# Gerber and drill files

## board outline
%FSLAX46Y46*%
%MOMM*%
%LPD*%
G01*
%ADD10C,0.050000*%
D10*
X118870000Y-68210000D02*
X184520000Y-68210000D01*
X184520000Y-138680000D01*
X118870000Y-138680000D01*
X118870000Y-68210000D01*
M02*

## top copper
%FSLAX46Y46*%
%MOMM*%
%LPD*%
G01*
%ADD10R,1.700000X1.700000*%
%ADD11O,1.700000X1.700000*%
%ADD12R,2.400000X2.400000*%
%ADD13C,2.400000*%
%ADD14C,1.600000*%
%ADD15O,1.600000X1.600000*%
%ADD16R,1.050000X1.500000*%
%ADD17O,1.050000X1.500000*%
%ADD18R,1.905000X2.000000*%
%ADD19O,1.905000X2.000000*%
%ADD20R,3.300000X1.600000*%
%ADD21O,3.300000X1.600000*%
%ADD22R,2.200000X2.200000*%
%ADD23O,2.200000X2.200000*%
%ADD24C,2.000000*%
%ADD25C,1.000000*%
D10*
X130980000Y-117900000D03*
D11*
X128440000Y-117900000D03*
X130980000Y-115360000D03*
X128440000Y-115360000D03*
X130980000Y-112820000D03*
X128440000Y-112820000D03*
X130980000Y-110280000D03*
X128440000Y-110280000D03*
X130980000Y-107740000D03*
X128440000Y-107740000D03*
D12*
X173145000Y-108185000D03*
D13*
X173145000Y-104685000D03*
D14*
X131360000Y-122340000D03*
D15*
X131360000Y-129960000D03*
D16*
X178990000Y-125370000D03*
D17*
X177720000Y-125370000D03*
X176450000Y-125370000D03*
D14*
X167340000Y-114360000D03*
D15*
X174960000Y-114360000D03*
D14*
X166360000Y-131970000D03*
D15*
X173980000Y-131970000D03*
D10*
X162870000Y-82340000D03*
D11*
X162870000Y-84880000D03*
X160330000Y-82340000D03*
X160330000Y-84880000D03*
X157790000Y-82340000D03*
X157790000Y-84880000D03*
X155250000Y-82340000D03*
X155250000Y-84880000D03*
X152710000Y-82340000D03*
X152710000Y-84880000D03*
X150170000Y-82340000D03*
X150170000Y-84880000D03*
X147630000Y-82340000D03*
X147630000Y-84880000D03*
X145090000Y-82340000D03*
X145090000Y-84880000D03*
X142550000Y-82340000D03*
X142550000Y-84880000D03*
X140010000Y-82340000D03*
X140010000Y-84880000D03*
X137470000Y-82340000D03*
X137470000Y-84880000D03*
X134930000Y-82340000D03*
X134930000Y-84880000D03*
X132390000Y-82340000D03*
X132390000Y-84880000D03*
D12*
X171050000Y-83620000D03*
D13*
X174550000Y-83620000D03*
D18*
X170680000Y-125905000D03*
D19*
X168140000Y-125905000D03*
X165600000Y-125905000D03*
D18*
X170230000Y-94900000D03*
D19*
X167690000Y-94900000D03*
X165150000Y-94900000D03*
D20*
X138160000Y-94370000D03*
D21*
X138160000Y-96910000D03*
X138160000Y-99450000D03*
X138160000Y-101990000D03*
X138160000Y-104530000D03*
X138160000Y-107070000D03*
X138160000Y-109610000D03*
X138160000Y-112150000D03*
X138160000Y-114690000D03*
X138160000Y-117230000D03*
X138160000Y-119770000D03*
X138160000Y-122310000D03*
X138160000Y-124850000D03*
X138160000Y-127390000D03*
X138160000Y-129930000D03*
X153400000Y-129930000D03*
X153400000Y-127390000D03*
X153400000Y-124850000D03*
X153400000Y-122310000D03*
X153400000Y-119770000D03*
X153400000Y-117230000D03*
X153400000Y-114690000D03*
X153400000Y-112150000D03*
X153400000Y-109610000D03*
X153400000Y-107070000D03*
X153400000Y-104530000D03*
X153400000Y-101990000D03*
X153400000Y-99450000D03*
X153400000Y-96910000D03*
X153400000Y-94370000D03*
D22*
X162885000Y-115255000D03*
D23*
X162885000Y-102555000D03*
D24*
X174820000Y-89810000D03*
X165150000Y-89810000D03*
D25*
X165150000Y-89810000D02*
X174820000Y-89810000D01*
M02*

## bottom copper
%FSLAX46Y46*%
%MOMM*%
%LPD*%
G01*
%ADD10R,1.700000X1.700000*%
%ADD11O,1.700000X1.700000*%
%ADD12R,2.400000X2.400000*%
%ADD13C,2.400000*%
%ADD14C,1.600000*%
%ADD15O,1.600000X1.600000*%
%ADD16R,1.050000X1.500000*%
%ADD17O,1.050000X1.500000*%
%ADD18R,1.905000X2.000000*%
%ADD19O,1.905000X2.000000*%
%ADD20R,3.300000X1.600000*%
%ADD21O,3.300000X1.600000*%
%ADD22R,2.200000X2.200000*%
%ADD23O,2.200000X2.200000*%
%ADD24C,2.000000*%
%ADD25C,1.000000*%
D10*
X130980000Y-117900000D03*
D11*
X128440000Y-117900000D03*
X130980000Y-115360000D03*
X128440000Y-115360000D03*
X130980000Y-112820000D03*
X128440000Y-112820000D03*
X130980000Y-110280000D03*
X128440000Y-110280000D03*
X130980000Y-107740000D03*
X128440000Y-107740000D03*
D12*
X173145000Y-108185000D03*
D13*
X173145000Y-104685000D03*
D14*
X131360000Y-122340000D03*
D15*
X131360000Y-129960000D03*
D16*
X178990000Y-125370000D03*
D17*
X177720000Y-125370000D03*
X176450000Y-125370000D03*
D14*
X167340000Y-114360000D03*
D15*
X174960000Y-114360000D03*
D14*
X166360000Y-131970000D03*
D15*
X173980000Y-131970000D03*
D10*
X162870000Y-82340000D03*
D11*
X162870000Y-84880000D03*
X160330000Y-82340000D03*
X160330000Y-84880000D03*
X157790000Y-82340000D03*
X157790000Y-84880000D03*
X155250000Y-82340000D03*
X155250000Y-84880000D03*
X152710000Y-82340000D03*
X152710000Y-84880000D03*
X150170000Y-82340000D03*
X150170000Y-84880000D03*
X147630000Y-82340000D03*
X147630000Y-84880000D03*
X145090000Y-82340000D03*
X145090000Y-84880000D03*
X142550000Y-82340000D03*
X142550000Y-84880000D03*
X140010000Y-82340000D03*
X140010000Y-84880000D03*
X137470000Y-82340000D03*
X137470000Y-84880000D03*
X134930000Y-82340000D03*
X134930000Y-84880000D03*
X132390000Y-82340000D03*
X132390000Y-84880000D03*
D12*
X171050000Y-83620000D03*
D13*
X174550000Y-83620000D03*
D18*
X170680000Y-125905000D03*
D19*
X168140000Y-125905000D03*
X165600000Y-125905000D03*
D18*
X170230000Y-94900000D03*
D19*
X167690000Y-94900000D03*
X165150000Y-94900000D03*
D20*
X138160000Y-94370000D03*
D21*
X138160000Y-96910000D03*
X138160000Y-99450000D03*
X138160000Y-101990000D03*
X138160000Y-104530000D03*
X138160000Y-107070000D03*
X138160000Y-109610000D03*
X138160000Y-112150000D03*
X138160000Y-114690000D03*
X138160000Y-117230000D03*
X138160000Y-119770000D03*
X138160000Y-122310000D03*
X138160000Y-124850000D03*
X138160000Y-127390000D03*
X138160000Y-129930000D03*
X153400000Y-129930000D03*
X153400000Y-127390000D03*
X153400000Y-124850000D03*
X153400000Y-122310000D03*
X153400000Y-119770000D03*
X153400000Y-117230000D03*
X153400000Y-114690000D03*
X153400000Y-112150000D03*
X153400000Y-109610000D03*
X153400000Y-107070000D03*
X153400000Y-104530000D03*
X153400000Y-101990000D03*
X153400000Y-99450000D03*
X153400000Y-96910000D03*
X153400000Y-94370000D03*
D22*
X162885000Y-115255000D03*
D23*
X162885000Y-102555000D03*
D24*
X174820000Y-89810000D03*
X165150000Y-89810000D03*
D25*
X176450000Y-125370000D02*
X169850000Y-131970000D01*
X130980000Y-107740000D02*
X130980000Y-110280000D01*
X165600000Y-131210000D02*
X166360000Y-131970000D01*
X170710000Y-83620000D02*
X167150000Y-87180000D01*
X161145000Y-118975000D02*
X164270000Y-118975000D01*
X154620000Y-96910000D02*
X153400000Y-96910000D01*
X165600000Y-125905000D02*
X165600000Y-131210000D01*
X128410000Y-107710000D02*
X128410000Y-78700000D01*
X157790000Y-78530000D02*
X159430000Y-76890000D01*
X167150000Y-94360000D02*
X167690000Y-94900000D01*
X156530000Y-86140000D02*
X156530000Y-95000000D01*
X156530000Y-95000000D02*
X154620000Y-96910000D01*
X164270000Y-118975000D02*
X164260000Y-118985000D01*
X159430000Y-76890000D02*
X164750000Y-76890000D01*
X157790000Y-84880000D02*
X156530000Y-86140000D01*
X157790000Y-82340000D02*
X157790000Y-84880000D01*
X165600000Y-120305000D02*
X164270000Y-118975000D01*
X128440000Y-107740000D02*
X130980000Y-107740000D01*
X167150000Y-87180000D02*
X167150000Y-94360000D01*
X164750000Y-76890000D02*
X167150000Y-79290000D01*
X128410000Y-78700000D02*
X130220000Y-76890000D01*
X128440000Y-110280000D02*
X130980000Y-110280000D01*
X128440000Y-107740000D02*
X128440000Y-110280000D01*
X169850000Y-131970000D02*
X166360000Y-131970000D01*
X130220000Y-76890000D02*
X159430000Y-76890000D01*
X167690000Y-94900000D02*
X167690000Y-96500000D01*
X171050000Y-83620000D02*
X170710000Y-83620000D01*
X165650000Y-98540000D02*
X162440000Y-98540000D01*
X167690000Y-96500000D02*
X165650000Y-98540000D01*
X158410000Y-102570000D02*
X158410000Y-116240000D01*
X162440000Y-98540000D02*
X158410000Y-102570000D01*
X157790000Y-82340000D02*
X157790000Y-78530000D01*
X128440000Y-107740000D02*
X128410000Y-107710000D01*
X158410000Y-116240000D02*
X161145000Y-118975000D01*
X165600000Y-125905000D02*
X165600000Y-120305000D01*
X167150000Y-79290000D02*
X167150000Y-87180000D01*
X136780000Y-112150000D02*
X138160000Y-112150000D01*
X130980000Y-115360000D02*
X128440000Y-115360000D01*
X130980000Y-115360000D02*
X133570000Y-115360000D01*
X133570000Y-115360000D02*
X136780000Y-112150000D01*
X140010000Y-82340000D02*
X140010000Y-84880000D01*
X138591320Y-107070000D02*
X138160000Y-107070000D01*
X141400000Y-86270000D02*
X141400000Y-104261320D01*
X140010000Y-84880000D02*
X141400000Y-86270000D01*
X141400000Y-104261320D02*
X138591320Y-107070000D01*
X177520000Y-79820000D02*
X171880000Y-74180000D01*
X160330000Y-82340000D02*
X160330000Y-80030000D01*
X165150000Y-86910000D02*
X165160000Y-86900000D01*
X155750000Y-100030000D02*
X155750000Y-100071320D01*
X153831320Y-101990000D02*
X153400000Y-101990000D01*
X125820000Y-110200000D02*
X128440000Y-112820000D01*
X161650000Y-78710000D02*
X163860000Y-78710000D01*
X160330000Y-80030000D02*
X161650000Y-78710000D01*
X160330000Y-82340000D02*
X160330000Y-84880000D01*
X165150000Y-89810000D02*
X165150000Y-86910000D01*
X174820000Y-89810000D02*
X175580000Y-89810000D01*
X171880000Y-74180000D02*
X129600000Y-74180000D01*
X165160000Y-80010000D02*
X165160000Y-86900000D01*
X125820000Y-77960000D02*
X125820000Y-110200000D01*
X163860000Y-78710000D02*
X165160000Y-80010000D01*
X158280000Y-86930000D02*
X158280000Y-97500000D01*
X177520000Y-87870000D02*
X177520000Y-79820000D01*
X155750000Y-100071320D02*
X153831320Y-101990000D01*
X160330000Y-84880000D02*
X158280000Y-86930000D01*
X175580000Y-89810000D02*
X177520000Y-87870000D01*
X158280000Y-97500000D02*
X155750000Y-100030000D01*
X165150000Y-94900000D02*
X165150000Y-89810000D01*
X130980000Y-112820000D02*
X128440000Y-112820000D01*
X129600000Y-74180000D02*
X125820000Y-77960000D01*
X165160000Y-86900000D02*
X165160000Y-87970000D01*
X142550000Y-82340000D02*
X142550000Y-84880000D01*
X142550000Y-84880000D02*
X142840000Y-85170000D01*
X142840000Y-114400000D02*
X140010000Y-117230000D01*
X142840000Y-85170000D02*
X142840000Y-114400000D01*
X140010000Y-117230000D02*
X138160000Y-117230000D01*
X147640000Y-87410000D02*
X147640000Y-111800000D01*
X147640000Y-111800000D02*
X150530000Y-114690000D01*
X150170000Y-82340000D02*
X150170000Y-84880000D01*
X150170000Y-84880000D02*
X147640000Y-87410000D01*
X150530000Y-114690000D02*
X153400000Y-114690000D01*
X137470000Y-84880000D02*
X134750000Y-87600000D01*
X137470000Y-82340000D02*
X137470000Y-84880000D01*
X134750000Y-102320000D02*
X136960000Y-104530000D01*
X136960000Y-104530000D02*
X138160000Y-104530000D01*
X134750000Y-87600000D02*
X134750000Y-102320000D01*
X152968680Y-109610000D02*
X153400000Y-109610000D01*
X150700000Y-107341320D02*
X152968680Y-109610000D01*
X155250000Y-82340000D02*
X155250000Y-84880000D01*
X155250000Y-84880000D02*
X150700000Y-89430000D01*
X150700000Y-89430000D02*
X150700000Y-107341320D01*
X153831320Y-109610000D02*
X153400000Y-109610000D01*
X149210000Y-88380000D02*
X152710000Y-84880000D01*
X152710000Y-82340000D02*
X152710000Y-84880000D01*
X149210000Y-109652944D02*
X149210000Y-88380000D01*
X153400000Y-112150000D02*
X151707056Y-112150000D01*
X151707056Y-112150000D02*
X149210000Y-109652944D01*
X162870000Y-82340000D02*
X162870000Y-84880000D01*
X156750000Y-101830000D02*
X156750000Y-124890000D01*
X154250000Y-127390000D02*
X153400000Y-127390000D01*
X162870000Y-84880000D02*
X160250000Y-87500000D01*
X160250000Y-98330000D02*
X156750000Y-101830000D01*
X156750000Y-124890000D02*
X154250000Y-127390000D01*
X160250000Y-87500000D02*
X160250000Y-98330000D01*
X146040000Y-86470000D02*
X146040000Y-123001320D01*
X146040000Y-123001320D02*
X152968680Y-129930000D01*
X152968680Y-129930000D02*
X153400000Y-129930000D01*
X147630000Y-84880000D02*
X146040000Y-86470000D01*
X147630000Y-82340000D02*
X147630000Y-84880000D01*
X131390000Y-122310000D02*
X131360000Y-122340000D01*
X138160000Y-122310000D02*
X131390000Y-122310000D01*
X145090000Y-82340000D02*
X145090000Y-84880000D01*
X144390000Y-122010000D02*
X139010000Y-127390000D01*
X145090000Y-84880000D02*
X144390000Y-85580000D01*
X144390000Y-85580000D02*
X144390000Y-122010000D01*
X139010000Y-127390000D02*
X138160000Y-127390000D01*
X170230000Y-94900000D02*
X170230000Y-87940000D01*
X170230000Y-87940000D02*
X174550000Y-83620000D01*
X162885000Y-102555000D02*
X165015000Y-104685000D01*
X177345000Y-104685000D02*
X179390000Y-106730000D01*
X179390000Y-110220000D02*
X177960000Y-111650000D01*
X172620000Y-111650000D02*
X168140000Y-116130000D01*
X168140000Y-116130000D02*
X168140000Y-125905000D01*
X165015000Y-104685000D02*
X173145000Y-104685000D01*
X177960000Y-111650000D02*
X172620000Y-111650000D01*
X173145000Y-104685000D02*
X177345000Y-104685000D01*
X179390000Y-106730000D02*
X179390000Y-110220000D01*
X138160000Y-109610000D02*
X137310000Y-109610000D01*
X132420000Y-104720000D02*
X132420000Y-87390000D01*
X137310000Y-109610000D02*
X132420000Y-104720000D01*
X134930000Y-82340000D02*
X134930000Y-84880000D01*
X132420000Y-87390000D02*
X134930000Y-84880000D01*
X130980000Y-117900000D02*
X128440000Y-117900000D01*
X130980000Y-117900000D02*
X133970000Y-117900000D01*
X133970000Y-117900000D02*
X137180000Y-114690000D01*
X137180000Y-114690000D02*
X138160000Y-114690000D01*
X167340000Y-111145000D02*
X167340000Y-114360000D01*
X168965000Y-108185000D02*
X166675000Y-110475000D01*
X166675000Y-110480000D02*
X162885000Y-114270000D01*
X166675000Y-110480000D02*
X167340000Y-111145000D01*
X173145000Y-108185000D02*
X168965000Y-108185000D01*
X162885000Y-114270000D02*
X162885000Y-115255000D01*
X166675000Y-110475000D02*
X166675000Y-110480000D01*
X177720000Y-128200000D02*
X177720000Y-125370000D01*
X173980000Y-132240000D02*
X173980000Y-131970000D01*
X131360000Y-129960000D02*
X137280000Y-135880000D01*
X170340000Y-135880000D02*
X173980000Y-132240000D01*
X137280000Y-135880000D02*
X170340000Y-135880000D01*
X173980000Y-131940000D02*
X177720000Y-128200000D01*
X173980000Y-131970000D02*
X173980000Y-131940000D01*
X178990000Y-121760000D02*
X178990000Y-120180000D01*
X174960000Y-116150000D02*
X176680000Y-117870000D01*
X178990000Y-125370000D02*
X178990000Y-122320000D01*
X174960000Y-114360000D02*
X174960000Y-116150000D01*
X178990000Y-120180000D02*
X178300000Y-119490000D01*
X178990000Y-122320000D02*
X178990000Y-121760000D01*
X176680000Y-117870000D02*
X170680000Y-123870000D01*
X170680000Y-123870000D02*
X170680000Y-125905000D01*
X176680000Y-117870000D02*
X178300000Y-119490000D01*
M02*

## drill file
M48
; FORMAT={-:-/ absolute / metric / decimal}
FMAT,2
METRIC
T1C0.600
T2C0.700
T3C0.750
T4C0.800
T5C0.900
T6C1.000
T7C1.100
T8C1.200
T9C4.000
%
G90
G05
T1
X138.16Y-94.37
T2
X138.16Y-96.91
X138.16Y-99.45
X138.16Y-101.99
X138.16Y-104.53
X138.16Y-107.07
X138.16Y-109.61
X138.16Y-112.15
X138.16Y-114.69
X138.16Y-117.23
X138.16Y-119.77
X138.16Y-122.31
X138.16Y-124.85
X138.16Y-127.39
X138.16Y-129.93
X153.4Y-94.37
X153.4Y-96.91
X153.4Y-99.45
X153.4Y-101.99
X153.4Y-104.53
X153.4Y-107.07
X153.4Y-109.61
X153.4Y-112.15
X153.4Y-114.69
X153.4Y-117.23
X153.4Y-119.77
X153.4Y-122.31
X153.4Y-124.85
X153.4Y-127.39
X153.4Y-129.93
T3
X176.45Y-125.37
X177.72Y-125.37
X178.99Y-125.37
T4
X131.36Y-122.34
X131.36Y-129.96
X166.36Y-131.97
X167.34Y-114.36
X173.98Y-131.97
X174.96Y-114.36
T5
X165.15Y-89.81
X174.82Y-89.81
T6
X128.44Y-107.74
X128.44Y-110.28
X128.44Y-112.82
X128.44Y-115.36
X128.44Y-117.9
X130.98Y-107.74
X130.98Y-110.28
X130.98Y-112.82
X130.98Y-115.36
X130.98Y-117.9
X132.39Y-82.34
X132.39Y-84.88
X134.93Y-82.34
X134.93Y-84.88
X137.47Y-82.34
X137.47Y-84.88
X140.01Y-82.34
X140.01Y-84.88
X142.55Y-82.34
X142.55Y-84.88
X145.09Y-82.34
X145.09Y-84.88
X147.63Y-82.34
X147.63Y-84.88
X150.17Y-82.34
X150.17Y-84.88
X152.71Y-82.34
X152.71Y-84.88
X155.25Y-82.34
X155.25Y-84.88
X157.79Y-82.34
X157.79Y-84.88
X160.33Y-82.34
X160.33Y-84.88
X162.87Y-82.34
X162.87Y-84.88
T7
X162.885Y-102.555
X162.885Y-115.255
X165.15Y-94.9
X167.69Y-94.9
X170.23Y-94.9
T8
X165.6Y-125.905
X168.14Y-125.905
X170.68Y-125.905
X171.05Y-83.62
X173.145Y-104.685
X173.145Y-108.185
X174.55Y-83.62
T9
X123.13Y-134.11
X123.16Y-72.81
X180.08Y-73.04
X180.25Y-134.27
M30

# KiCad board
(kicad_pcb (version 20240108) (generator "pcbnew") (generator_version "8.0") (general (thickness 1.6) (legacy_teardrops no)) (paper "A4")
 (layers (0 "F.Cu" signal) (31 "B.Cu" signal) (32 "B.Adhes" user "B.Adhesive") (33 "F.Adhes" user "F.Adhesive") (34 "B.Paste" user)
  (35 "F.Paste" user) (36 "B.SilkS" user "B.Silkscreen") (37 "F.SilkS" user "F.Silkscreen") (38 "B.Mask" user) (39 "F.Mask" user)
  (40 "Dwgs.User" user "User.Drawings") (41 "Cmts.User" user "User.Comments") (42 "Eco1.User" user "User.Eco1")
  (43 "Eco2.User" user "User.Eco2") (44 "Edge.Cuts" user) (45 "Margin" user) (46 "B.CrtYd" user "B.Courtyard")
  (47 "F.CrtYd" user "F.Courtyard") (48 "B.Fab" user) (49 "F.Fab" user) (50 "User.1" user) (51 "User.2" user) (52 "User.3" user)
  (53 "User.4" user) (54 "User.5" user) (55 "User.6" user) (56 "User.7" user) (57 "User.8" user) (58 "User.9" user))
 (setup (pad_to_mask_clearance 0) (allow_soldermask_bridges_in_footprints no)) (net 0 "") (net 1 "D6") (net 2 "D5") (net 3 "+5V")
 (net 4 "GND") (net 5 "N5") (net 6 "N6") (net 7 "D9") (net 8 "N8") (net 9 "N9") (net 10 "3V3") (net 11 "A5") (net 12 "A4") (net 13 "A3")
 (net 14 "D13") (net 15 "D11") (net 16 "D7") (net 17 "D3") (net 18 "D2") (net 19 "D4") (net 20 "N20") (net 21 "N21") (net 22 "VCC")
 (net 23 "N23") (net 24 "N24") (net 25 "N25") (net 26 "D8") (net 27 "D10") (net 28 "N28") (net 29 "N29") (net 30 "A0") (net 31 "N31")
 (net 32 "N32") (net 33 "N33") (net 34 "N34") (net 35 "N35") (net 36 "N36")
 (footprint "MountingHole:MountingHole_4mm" (layer "F.Cu") (at 180.25 134.27)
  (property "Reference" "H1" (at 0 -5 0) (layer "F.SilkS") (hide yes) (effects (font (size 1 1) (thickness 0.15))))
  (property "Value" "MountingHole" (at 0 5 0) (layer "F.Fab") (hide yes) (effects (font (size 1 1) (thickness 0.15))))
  (pad "" np_thru_hole circle (at 0 0) (size 4 4) (drill 4) (layers "*.Cu" "*.Mask")))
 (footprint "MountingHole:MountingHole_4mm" (layer "F.Cu") (at 123.16 72.81)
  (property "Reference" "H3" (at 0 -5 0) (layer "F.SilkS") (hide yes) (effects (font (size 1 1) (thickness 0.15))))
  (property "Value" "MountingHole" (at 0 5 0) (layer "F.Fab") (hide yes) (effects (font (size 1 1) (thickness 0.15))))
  (pad "" np_thru_hole circle (at 0 0) (size 4 4) (drill 4) (layers "*.Cu" "*.Mask")))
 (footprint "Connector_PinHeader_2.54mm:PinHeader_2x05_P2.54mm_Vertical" (layer "F.Cu") (at 130.98 117.9 180)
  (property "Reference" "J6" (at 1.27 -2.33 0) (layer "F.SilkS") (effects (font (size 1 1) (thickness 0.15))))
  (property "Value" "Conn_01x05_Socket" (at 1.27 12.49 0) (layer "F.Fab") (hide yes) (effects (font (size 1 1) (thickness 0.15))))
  (pad "1" thru_hole rect (at 0 0 180) (size 1.7 1.7) (drill 1) (layers "*.Cu" "*.Mask") (remove_unused_layers no) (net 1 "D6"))
  (pad "1" thru_hole oval (at 2.54 0 180) (size 1.7 1.7) (drill 1) (layers "*.Cu" "*.Mask") (remove_unused_layers no) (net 1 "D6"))
  (pad "2" thru_hole oval (at 0 2.54 180) (size 1.7 1.7) (drill 1) (layers "*.Cu" "*.Mask") (remove_unused_layers no) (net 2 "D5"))
  (pad "2" thru_hole oval (at 2.54 2.54 180) (size 1.7 1.7) (drill 1) (layers "*.Cu" "*.Mask") (remove_unused_layers no) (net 2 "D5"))
  (pad "3" thru_hole oval (at 0 5.08 180) (size 1.7 1.7) (drill 1) (layers "*.Cu" "*.Mask") (remove_unused_layers no) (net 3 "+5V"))
  (pad "3" thru_hole oval (at 2.54 5.08 180) (size 1.7 1.7) (drill 1) (layers "*.Cu" "*.Mask") (remove_unused_layers no) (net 3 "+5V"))
  (pad "4" thru_hole oval (at 0 7.62 180) (size 1.7 1.7) (drill 1) (layers "*.Cu" "*.Mask") (remove_unused_layers no) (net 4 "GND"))
  (pad "4" thru_hole oval (at 2.54 7.62 180) (size 1.7 1.7) (drill 1) (layers "*.Cu" "*.Mask") (remove_unused_layers no) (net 4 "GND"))
  (pad "5" thru_hole oval (at 0 10.16 180) (size 1.7 1.7) (drill 1) (layers "*.Cu" "*.Mask") (remove_unused_layers no) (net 4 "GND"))
  (pad "5" thru_hole oval (at 2.54 10.16 180) (size 1.7 1.7) (drill 1) (layers "*.Cu" "*.Mask") (remove_unused_layers no) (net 4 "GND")))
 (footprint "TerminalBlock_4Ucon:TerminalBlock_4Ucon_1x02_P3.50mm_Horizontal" (layer "F.Cu") (at 173.145 108.185 90)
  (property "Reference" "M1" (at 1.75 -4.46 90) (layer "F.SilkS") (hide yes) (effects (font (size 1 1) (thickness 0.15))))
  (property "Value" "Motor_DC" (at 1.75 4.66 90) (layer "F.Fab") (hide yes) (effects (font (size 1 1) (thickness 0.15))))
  (pad "1" thru_hole rect (at 0 0 90) (size 2.4 2.4) (drill 1.2) (layers "*.Cu" "*.Mask") (remove_unused_layers no) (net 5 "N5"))
  (pad "2" thru_hole circle (at 3.5 0 90) (size 2.4 2.4) (drill 1.2) (layers "*.Cu" "*.Mask") (remove_unused_layers no) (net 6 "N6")))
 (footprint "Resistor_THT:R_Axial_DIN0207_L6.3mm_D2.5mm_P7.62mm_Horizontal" (layer "F.Cu") (at 131.36 122.34 -90)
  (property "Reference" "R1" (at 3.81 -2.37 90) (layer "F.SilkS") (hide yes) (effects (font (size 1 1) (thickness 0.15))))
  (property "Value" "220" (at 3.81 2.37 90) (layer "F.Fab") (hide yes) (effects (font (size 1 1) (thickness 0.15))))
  (pad "1" thru_hole circle (at 0 0 270) (size 1.6 1.6) (drill 0.8) (layers "*.Cu" "*.Mask") (remove_unused_layers no) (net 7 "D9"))
  (pad "2" thru_hole oval (at 7.62 0 270) (size 1.6 1.6) (drill 0.8) (layers "*.Cu" "*.Mask") (remove_unused_layers no) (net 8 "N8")))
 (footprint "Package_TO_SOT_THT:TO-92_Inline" (layer "F.Cu") (at 178.99 125.37 180)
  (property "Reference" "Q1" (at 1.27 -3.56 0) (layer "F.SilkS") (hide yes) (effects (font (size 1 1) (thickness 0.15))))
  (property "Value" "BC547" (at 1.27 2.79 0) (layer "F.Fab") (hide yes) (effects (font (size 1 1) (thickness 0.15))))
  (pad "1" thru_hole rect (at 0 0 180) (size 1.05 1.5) (drill 0.75) (layers "*.Cu" "*.Mask") (remove_unused_layers no) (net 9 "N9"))
  (pad "2" thru_hole oval (at 1.27 0 180) (size 1.05 1.5) (drill 0.75) (layers "*.Cu" "*.Mask") (remove_unused_layers no) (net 8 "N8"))
  (pad "3" thru_hole oval (at 2.54 0 180) (size 1.05 1.5) (drill 0.75) (layers "*.Cu" "*.Mask") (remove_unused_layers no) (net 4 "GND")))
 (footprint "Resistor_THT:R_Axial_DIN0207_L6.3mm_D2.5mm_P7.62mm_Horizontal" (layer "F.Cu") (at 167.34 114.36)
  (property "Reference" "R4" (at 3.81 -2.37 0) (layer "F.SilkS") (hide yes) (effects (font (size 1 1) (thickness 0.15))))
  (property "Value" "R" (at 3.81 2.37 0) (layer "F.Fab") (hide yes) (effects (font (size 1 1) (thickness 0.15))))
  (pad "1" thru_hole circle (at 0 0) (size 1.6 1.6) (drill 0.8) (layers "*.Cu" "*.Mask") (remove_unused_layers no) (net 5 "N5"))
  (pad "2" thru_hole oval (at 7.62 0) (size 1.6 1.6) (drill 0.8) (layers "*.Cu" "*.Mask") (remove_unused_layers no) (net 9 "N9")))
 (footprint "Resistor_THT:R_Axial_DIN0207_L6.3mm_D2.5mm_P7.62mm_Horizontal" (layer "F.Cu") (at 166.36 131.97)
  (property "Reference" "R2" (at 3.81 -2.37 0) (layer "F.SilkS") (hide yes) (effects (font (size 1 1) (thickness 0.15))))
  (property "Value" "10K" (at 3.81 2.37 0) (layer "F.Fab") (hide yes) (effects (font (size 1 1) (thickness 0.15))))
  (pad "1" thru_hole circle (at 0 0) (size 1.6 1.6) (drill 0.8) (layers "*.Cu" "*.Mask") (remove_unused_layers no) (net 4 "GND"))
  (pad "2" thru_hole oval (at 7.62 0) (size 1.6 1.6) (drill 0.8) (layers "*.Cu" "*.Mask") (remove_unused_layers no) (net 8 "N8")))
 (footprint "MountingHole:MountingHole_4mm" (layer "F.Cu") (at 123.13 134.11)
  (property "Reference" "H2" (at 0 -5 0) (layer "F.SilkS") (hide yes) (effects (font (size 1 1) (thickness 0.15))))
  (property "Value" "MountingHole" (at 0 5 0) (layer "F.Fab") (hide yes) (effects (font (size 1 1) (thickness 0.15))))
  (pad "" np_thru_hole circle (at 0 0) (size 4 4) (drill 4) (layers "*.Cu" "*.Mask")))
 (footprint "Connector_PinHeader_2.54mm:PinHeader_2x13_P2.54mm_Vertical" (layer "F.Cu") (at 162.87 82.34 -90)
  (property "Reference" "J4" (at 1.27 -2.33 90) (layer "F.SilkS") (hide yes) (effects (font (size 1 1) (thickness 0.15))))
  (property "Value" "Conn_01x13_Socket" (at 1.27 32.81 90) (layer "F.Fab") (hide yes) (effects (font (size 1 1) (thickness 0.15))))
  (pad "1" thru_hole rect (at 0 0 270) (size 1.7 1.7) (drill 1) (layers "*.Cu" "*.Mask") (remove_unused_layers no) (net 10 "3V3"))
  (pad "1" thru_hole oval (at 2.54 0 270) (size 1.7 1.7) (drill 1) (layers "*.Cu" "*.Mask") (remove_unused_layers no) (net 10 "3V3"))
  (pad "2" thru_hole oval (at 0 2.54 270) (size 1.7 1.7) (drill 1) (layers "*.Cu" "*.Mask") (remove_unused_layers no) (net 3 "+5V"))
  (pad "2" thru_hole oval (at 2.54 2.54 270) (size 1.7 1.7) (drill 1) (layers "*.Cu" "*.Mask") (remove_unused_layers no) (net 3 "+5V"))
  (pad "3" thru_hole oval (at 0 5.08 270) (size 1.7 1.7) (drill 1) (layers "*.Cu" "*.Mask") (remove_unused_layers no) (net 4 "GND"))
  (pad "3" thru_hole oval (at 2.54 5.08 270) (size 1.7 1.7) (drill 1) (layers "*.Cu" "*.Mask") (remove_unused_layers no) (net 4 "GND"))
  (pad "4" thru_hole oval (at 0 7.62 270) (size 1.7 1.7) (drill 1) (layers "*.Cu" "*.Mask") (remove_unused_layers no) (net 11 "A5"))
  (pad "4" thru_hole oval (at 2.54 7.62 270) (size 1.7 1.7) (drill 1) (layers "*.Cu" "*.Mask") (remove_unused_layers no) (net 11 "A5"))
  (pad "5" thru_hole oval (at 0 10.16 270) (size 1.7 1.7) (drill 1) (layers "*.Cu" "*.Mask") (remove_unused_layers no) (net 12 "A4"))
  (pad "5" thru_hole oval (at 2.54 10.16 270) (size 1.7 1.7) (drill 1) (layers "*.Cu" "*.Mask") (remove_unused_layers no) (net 12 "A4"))
  (pad "6" thru_hole oval (at 0 12.7 270) (size 1.7 1.7) (drill 1) (layers "*.Cu" "*.Mask") (remove_unused_layers no) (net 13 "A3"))
  (pad "6" thru_hole oval (at 2.54 12.7 270) (size 1.7 1.7) (drill 1) (layers "*.Cu" "*.Mask") (remove_unused_layers no) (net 13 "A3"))
  (pad "7" thru_hole oval (at 0 15.24 270) (size 1.7 1.7) (drill 1) (layers "*.Cu" "*.Mask") (remove_unused_layers no) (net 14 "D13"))
  (pad "7" thru_hole oval (at 2.54 15.24 270) (size 1.7 1.7) (drill 1) (layers "*.Cu" "*.Mask") (remove_unused_layers no) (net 14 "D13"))
  (pad "8" thru_hole oval (at 0 17.78 270) (size 1.7 1.7) (drill 1) (layers "*.Cu" "*.Mask") (remove_unused_layers no) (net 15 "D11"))
  (pad "8" thru_hole oval (at 2.54 17.78 270) (size 1.7 1.7) (drill 1) (layers "*.Cu" "*.Mask") (remove_unused_layers no) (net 15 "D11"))
  (pad "9" thru_hole oval (at 0 20.32 270) (size 1.7 1.7) (drill 1) (layers "*.Cu" "*.Mask") (remove_unused_layers no) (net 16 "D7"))
  (pad "9" thru_hole oval (at 2.54 20.32 270) (size 1.7 1.7) (drill 1) (layers "*.Cu" "*.Mask") (remove_unused_layers no) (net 16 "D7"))
  (pad "10" thru_hole oval (at 0 22.86 270) (size 1.7 1.7) (drill 1) (layers "*.Cu" "*.Mask") (remove_unused_layers no) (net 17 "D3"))
  (pad "10" thru_hole oval (at 2.54 22.86 270) (size 1.7 1.7) (drill 1) (layers "*.Cu" "*.Mask") (remove_unused_layers no) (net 17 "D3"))
  (pad "11" thru_hole oval (at 0 25.4 270) (size 1.7 1.7) (drill 1) (layers "*.Cu" "*.Mask") (remove_unused_layers no) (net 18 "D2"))
  (pad "11" thru_hole oval (at 2.54 25.4 270) (size 1.7 1.7) (drill 1) (layers "*.Cu" "*.Mask") (remove_unused_layers no) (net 18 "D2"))
  (pad "12" thru_hole oval (at 0 27.94 270) (size 1.7 1.7) (drill 1) (layers "*.Cu" "*.Mask") (remove_unused_layers no) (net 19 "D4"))
  (pad "12" thru_hole oval (at 2.54 27.94 270) (size 1.7 1.7) (drill 1) (layers "*.Cu" "*.Mask") (remove_unused_layers no) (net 19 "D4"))
  (pad "13" thru_hole oval (at 0 30.48 270) (size 1.7 1.7) (drill 1) (layers "*.Cu" "*.Mask") (remove_unused_layers no) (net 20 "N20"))
  (pad "13" thru_hole oval (at 2.54 30.48 270) (size 1.7 1.7) (drill 1) (layers "*.Cu" "*.Mask") (remove_unused_layers no) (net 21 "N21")))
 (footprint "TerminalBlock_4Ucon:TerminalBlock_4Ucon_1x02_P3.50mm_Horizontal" (layer "F.Cu") (at 171.05 83.62)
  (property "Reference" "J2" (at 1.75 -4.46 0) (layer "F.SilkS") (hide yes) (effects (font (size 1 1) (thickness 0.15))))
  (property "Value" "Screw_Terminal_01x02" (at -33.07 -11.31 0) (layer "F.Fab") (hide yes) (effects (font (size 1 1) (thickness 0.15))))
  (pad "1" thru_hole rect (at 0 0) (size 2.4 2.4) (drill 1.2) (layers "*.Cu" "*.Mask") (remove_unused_layers no) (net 4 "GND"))
  (pad "2" thru_hole circle (at 3.5 0) (size 2.4 2.4) (drill 1.2) (layers "*.Cu" "*.Mask") (remove_unused_layers no) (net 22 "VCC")))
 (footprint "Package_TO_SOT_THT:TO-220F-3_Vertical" (layer "F.Cu") (at 170.68 125.905 180)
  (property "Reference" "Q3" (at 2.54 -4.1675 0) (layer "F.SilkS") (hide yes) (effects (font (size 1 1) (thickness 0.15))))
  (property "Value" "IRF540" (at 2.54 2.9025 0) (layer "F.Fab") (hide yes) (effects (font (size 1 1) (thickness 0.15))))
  (pad "1" thru_hole rect (at 0 0 180) (size 1.905 2) (drill 1.2) (layers "*.Cu" "*.Mask") (remove_unused_layers no) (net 9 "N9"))
  (pad "2" thru_hole oval (at 2.54 0 180) (size 1.905 2) (drill 1.2) (layers "*.Cu" "*.Mask") (remove_unused_layers no) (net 6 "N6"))
  (pad "3" thru_hole oval (at 5.08 0 180) (size 1.905 2) (drill 1.2) (layers "*.Cu" "*.Mask") (remove_unused_layers no) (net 4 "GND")))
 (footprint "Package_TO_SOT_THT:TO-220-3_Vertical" (layer "F.Cu") (at 170.23 94.9 180)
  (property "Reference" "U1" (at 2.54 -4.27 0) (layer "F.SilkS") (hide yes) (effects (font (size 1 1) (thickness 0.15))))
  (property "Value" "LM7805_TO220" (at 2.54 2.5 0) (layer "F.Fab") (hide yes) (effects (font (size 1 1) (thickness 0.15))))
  (pad "1" thru_hole rect (at 0 0 180) (size 1.905 2) (drill 1.1) (layers "*.Cu" "*.Mask") (remove_unused_layers no) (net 22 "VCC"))
  (pad "2" thru_hole oval (at 2.54 0 180) (size 1.905 2) (drill 1.1) (layers "*.Cu" "*.Mask") (remove_unused_layers no) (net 4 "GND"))
  (pad "3" thru_hole oval (at 5.08 0 180) (size 1.905 2) (drill 1.1) (layers "*.Cu" "*.Mask") (remove_unused_layers no) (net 3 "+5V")))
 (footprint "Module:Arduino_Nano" (layer "F.Cu") (at 138.16 94.37)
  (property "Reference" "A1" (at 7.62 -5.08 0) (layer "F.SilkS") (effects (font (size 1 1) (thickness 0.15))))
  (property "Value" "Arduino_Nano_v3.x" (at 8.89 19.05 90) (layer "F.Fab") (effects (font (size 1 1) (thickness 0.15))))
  (pad "1" thru_hole rect (at 0 0) (size 3.3 1.6) (drill 0.6) (layers "*.Cu" "*.Mask") (remove_unused_layers no) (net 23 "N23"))
  (pad "2" thru_hole oval (at 0 2.54) (size 3.3 1.6) (drill 0.7) (layers "*.Cu" "*.Mask") (remove_unused_layers no) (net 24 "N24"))
  (pad "3" thru_hole oval (at 0 5.08) (size 3.3 1.6) (drill 0.7) (layers "*.Cu" "*.Mask") (remove_unused_layers no) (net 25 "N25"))
  (pad "4" thru_hole oval (at 0 7.62) (size 3.3 1.6) (drill 0.7) (layers "*.Cu" "*.Mask") (remove_unused_layers no) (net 4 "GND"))
  (pad "5" thru_hole oval (at 0 10.16) (size 3.3 1.6) (drill 0.7) (layers "*.Cu" "*.Mask") (remove_unused_layers no) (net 18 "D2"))
  (pad "6" thru_hole oval (at 0 12.7) (size 3.3 1.6) (drill 0.7) (layers "*.Cu" "*.Mask") (remove_unused_layers no) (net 17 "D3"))
  (pad "7" thru_hole oval (at 0 15.24) (size 3.3 1.6) (drill 0.7) (layers "*.Cu" "*.Mask") (remove_unused_layers no) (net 19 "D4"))
  (pad "8" thru_hole oval (at 0 17.78) (size 3.3 1.6) (drill 0.7) (layers "*.Cu" "*.Mask") (remove_unused_layers no) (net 2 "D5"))
  (pad "9" thru_hole oval (at 0 20.32) (size 3.3 1.6) (drill 0.7) (layers "*.Cu" "*.Mask") (remove_unused_layers no) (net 1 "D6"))
  (pad "10" thru_hole oval (at 0 22.86) (size 3.3 1.6) (drill 0.7) (layers "*.Cu" "*.Mask") (remove_unused_layers no) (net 16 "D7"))
  (pad "11" thru_hole oval (at 0 25.4) (size 3.3 1.6) (drill 0.7) (layers "*.Cu" "*.Mask") (remove_unused_layers no) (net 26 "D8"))
  (pad "12" thru_hole oval (at 0 27.94) (size 3.3 1.6) (drill 0.7) (layers "*.Cu" "*.Mask") (remove_unused_layers no) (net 7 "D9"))
  (pad "13" thru_hole oval (at 0 30.48) (size 3.3 1.6) (drill 0.7) (layers "*.Cu" "*.Mask") (remove_unused_layers no) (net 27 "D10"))
  (pad "14" thru_hole oval (at 0 33.02) (size 3.3 1.6) (drill 0.7) (layers "*.Cu" "*.Mask") (remove_unused_layers no) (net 15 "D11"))
  (pad "15" thru_hole oval (at 0 35.56) (size 3.3 1.6) (drill 0.7) (layers "*.Cu" "*.Mask") (remove_unused_layers no) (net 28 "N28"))
  (pad "16" thru_hole oval (at 15.24 35.56) (size 3.3 1.6) (drill 0.7) (layers "*.Cu" "*.Mask") (remove_unused_layers no) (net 14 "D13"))
  (pad "17" thru_hole oval (at 15.24 33.02) (size 3.3 1.6) (drill 0.7) (layers "*.Cu" "*.Mask") (remove_unused_layers no) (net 10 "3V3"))
  (pad "18" thru_hole oval (at 15.24 30.48) (size 3.3 1.6) (drill 0.7) (layers "*.Cu" "*.Mask") (remove_unused_layers no) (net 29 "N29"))
  (pad "19" thru_hole oval (at 15.24 27.94) (size 3.3 1.6) (drill 0.7) (layers "*.Cu" "*.Mask") (remove_unused_layers no) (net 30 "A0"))
  (pad "20" thru_hole oval (at 15.24 25.4) (size 3.3 1.6) (drill 0.7) (layers "*.Cu" "*.Mask") (remove_unused_layers no) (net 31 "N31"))
  (pad "21" thru_hole oval (at 15.24 22.86) (size 3.3 1.6) (drill 0.7) (layers "*.Cu" "*.Mask") (remove_unused_layers no) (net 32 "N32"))
  (pad "22" thru_hole oval (at 15.24 20.32) (size 3.3 1.6) (drill 0.7) (layers "*.Cu" "*.Mask") (remove_unused_layers no) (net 13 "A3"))
  (pad "23" thru_hole oval (at 15.24 17.78) (size 3.3 1.6) (drill 0.7) (layers "*.Cu" "*.Mask") (remove_unused_layers no) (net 12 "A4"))
  (pad "24" thru_hole oval (at 15.24 15.24) (size 3.3 1.6) (drill 0.7) (layers "*.Cu" "*.Mask") (remove_unused_layers no) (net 11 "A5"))
  (pad "25" thru_hole oval (at 15.24 12.7) (size 3.3 1.6) (drill 0.7) (layers "*.Cu" "*.Mask") (remove_unused_layers no) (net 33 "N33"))
  (pad "26" thru_hole oval (at 15.24 10.16) (size 3.3 1.6) (drill 0.7) (layers "*.Cu" "*.Mask") (remove_unused_layers no) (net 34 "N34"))
  (pad "27" thru_hole oval (at 15.24 7.62) (size 3.3 1.6) (drill 0.7) (layers "*.Cu" "*.Mask") (remove_unused_layers no) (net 3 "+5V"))
  (pad "28" thru_hole oval (at 15.24 5.08) (size 3.3 1.6) (drill 0.7) (layers "*.Cu" "*.Mask") (remove_unused_layers no) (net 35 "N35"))
  (pad "29" thru_hole oval (at 15.24 2.54) (size 3.3 1.6) (drill 0.7) (layers "*.Cu" "*.Mask") (remove_unused_layers no) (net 4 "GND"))
  (pad "30" thru_hole oval (at 15.24 0) (size 3.3 1.6) (drill 0.7) (layers "*.Cu" "*.Mask") (remove_unused_layers no) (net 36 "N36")))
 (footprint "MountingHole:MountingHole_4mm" (layer "F.Cu") (at 180.08 73.04)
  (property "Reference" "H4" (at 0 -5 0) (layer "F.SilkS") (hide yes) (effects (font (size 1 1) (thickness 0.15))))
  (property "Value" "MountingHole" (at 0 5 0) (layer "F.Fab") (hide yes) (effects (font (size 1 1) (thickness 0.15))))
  (pad "" np_thru_hole circle (at 0 0) (size 4 4) (drill 4) (layers "*.Cu" "*.Mask")))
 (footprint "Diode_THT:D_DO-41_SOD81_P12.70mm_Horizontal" (layer "F.Cu") (at 162.885 115.255 90)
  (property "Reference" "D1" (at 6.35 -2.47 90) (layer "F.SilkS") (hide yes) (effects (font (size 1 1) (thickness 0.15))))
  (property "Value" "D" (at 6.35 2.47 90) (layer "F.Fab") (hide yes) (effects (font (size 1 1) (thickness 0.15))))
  (pad "1" thru_hole rect (at 0 0 90) (size 2.2 2.2) (drill 1.1) (layers "*.Cu" "*.Mask") (remove_unused_layers no) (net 5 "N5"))
  (pad "2" thru_hole oval (at 12.7 0 90) (size 2.2 2.2) (drill 1.1) (layers "*.Cu" "*.Mask") (remove_unused_layers no) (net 6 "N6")))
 (gr_rect (start 118.87 68.21) (end 184.52 138.68) (stroke (width 0.05) (type default)) (fill none) (layer "Edge.Cuts"))
 (segment (start 176.45 125.37) (end 169.85 131.97) (width 1) (layer "B.Cu") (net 4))
 (segment (start 130.98 107.74) (end 130.98 110.28) (width 1) (layer "B.Cu") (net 4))
 (segment (start 165.6 131.21) (end 166.36 131.97) (width 1) (layer "B.Cu") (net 4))
 (segment (start 170.71 83.62) (end 167.15 87.18) (width 1) (layer "B.Cu") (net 4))
 (segment (start 161.145 118.975) (end 164.27 118.975) (width 1) (layer "B.Cu") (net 4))
 (segment (start 154.62 96.91) (end 153.4 96.91) (width 1) (layer "B.Cu") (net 4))
 (segment (start 165.6 125.905) (end 165.6 131.21) (width 1) (layer "B.Cu") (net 4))
 (segment (start 128.41 107.71) (end 128.41 78.7) (width 1) (layer "B.Cu") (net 4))
 (segment (start 157.79 78.53) (end 159.43 76.89) (width 1) (layer "B.Cu") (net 4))
 (segment (start 167.15 94.36) (end 167.69 94.9) (width 1) (layer "B.Cu") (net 4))
 (segment (start 156.53 86.14) (end 156.53 95) (width 1) (layer "B.Cu") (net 4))
 (segment (start 156.53 95) (end 154.62 96.91) (width 1) (layer "B.Cu") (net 4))
 (segment (start 164.27 118.975) (end 164.26 118.985) (width 1) (layer "B.Cu") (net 4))
 (segment (start 159.43 76.89) (end 164.75 76.89) (width 1) (layer "B.Cu") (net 4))
 (segment (start 157.79 84.88) (end 156.53 86.14) (width 1) (layer "B.Cu") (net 4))
 (segment (start 157.79 82.34) (end 157.79 84.88) (width 1) (layer "B.Cu") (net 4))
 (segment (start 165.6 120.305) (end 164.27 118.975) (width 1) (layer "B.Cu") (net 4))
 (segment (start 128.44 107.74) (end 130.98 107.74) (width 1) (layer "B.Cu") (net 4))
 (segment (start 167.15 87.18) (end 167.15 94.36) (width 1) (layer "B.Cu") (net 4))
 (segment (start 164.75 76.89) (end 167.15 79.29) (width 1) (layer "B.Cu") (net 4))
 (segment (start 128.41 78.7) (end 130.22 76.89) (width 1) (layer "B.Cu") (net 4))
 (segment (start 128.44 110.28) (end 130.98 110.28) (width 1) (layer "B.Cu") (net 4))
 (segment (start 128.44 107.74) (end 128.44 110.28) (width 1) (layer "B.Cu") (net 4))
 (segment (start 169.85 131.97) (end 166.36 131.97) (width 1) (layer "B.Cu") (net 4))
 (segment (start 130.22 76.89) (end 159.43 76.89) (width 1) (layer "B.Cu") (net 4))
 (segment (start 167.69 94.9) (end 167.69 96.5) (width 1) (layer "B.Cu") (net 4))
 (segment (start 171.05 83.62) (end 170.71 83.62) (width 1) (layer "B.Cu") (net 4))
 (segment (start 165.65 98.54) (end 162.44 98.54) (width 1) (layer "B.Cu") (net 4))
 (segment (start 167.69 96.5) (end 165.65 98.54) (width 1) (layer "B.Cu") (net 4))
 (segment (start 158.41 102.57) (end 158.41 116.24) (width 1) (layer "B.Cu") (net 4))
 (segment (start 162.44 98.54) (end 158.41 102.57) (width 1) (layer "B.Cu") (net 4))
 (segment (start 157.79 82.34) (end 157.79 78.53) (width 1) (layer "B.Cu") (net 4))
 (segment (start 128.44 107.74) (end 128.41 107.71) (width 1) (layer "B.Cu") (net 4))
 (segment (start 158.41 116.24) (end 161.145 118.975) (width 1) (layer "B.Cu") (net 4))
 (segment (start 165.6 125.905) (end 165.6 120.305) (width 1) (layer "B.Cu") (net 4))
 (segment (start 167.15 79.29) (end 167.15 87.18) (width 1) (layer "B.Cu") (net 4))
 (segment (start 136.78 112.15) (end 138.16 112.15) (width 1) (layer "B.Cu") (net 2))
 (segment (start 130.98 115.36) (end 128.44 115.36) (width 1) (layer "B.Cu") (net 2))
 (segment (start 130.98 115.36) (end 133.57 115.36) (width 1) (layer "B.Cu") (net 2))
 (segment (start 133.57 115.36) (end 136.78 112.15) (width 1) (layer "B.Cu") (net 2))
 (segment (start 140.01 82.34) (end 140.01 84.88) (width 1) (layer "B.Cu") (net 17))
 (segment (start 138.59132 107.07) (end 138.16 107.07) (width 1) (layer "B.Cu") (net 17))
 (segment (start 141.4 86.27) (end 141.4 104.26132) (width 1) (layer "B.Cu") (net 17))
 (segment (start 140.01 84.88) (end 141.4 86.27) (width 1) (layer "B.Cu") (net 17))
 (segment (start 141.4 104.26132) (end 138.59132 107.07) (width 1) (layer "B.Cu") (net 17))
 (segment (start 165.15 89.81) (end 174.82 89.81) (width 1) (layer "F.Cu") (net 3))
 (via micro (at 174.82 89.81) (size 2) (drill 0.9) (layers "F.Cu" "B.Cu") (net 3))
 (via micro (at 165.15 89.81) (size 2) (drill 0.9) (layers "F.Cu" "B.Cu") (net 3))
 (segment (start 177.52 79.82) (end 171.88 74.18) (width 1) (layer "B.Cu") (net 3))
 (segment (start 160.33 82.34) (end 160.33 80.03) (width 1) (layer "B.Cu") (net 3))
 (segment (start 165.15 86.91) (end 165.16 86.9) (width 1) (layer "B.Cu") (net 3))
 (segment (start 155.75 100.03) (end 155.75 100.07132) (width 1) (layer "B.Cu") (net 3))
 (segment (start 153.83132 101.99) (end 153.4 101.99) (width 1) (layer "B.Cu") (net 3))
 (segment (start 125.82 110.2) (end 128.44 112.82) (width 1) (layer "B.Cu") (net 3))
 (segment (start 161.65 78.71) (end 163.86 78.71) (width 1) (layer "B.Cu") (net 3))
 (segment (start 160.33 80.03) (end 161.65 78.71) (width 1) (layer "B.Cu") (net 3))
 (segment (start 160.33 82.34) (end 160.33 84.88) (width 1) (layer "B.Cu") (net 3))
 (segment (start 165.15 89.81) (end 165.15 86.91) (width 1) (layer "B.Cu") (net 3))
 (segment (start 174.82 89.81) (end 175.58 89.81) (width 1) (layer "B.Cu") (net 3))
 (segment (start 171.88 74.18) (end 129.6 74.18) (width 1) (layer "B.Cu") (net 3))
 (segment (start 165.16 80.01) (end 165.16 86.9) (width 1) (layer "B.Cu") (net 3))
 (segment (start 125.82 77.96) (end 125.82 110.2) (width 1) (layer "B.Cu") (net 3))
 (segment (start 163.86 78.71) (end 165.16 80.01) (width 1) (layer "B.Cu") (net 3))
 (segment (start 158.28 86.93) (end 158.28 97.5) (width 1) (layer "B.Cu") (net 3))
 (segment (start 177.52 87.87) (end 177.52 79.82) (width 1) (layer "B.Cu") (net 3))
 (segment (start 155.75 100.07132) (end 153.83132 101.99) (width 1) (layer "B.Cu") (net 3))
 (segment (start 160.33 84.88) (end 158.28 86.93) (width 1) (layer "B.Cu") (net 3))
 (segment (start 175.58 89.81) (end 177.52 87.87) (width 1) (layer "B.Cu") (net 3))
 (segment (start 158.28 97.5) (end 155.75 100.03) (width 1) (layer "B.Cu") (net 3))
 (segment (start 165.15 94.9) (end 165.15 89.81) (width 1) (layer "B.Cu") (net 3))
 (segment (start 130.98 112.82) (end 128.44 112.82) (width 1) (layer "B.Cu") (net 3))
 (segment (start 129.6 74.18) (end 125.82 77.96) (width 1) (layer "B.Cu") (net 3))
 (segment (start 165.16 86.9) (end 165.16 87.97) (width 1) (layer "B.Cu") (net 3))
 (segment (start 142.55 82.34) (end 142.55 84.88) (width 1) (layer "B.Cu") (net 16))
 (segment (start 142.55 84.88) (end 142.84 85.17) (width 1) (layer "B.Cu") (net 16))
 (segment (start 142.84 114.4) (end 140.01 117.23) (width 1) (layer "B.Cu") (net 16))
 (segment (start 142.84 85.17) (end 142.84 114.4) (width 1) (layer "B.Cu") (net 16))
 (segment (start 140.01 117.23) (end 138.16 117.23) (width 1) (layer "B.Cu") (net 16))
 (segment (start 147.64 87.41) (end 147.64 111.8) (width 1) (layer "B.Cu") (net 13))
 (segment (start 147.64 111.8) (end 150.53 114.69) (width 1) (layer "B.Cu") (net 13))
 (segment (start 150.17 82.34) (end 150.17 84.88) (width 1) (layer "B.Cu") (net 13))
 (segment (start 150.17 84.88) (end 147.64 87.41) (width 1) (layer "B.Cu") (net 13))
 (segment (start 150.53 114.69) (end 153.4 114.69) (width 1) (layer "B.Cu") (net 13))
 (segment (start 137.47 84.88) (end 134.75 87.6) (width 1) (layer "B.Cu") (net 18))
 (segment (start 137.47 82.34) (end 137.47 84.88) (width 1) (layer "B.Cu") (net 18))
 (segment (start 134.75 102.32) (end 136.96 104.53) (width 1) (layer "B.Cu") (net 18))
 (segment (start 136.96 104.53) (end 138.16 104.53) (width 1) (layer "B.Cu") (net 18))
 (segment (start 134.75 87.6) (end 134.75 102.32) (width 1) (layer "B.Cu") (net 18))
 (segment (start 152.96868 109.61) (end 153.4 109.61) (width 1) (layer "B.Cu") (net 11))
 (segment (start 150.7 107.34132) (end 152.96868 109.61) (width 1) (layer "B.Cu") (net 11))
 (segment (start 155.25 82.34) (end 155.25 84.88) (width 1) (layer "B.Cu") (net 11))
 (segment (start 155.25 84.88) (end 150.7 89.43) (width 1) (layer "B.Cu") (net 11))
 (segment (start 150.7 89.43) (end 150.7 107.34132) (width 1) (layer "B.Cu") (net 11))
 (segment (start 153.83132 109.61) (end 153.4 109.61) (width 1) (layer "B.Cu") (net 11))
 (segment (start 149.21 88.38) (end 152.71 84.88) (width 1) (layer "B.Cu") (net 12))
 (segment (start 152.71 82.34) (end 152.71 84.88) (width 1) (layer "B.Cu") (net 12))
 (segment (start 149.21 109.652944) (end 149.21 88.38) (width 1) (layer "B.Cu") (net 12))
 (segment (start 153.4 112.15) (end 151.707056 112.15) (width 1) (layer "B.Cu") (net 12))
 (segment (start 151.707056 112.15) (end 149.21 109.652944) (width 1) (layer "B.Cu") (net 12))
 (segment (start 162.87 82.34) (end 162.87 84.88) (width 1) (layer "B.Cu") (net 10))
 (segment (start 156.75 101.83) (end 156.75 124.89) (width 1) (layer "B.Cu") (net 10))
 (segment (start 154.25 127.39) (end 153.4 127.39) (width 1) (layer "B.Cu") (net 10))
 (segment (start 162.87 84.88) (end 160.25 87.5) (width 1) (layer "B.Cu") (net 10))
 (segment (start 160.25 98.33) (end 156.75 101.83) (width 1) (layer "B.Cu") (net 10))
 (segment (start 156.75 124.89) (end 154.25 127.39) (width 1) (layer "B.Cu") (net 10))
 (segment (start 160.25 87.5) (end 160.25 98.33) (width 1) (layer "B.Cu") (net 10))
 (segment (start 146.04 86.47) (end 146.04 123.00132) (width 1) (layer "B.Cu") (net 14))
 (segment (start 146.04 123.00132) (end 152.96868 129.93) (width 1) (layer "B.Cu") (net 14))
 (segment (start 152.96868 129.93) (end 153.4 129.93) (width 1) (layer "B.Cu") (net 14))
 (segment (start 147.63 84.88) (end 146.04 86.47) (width 1) (layer "B.Cu") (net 14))
 (segment (start 147.63 82.34) (end 147.63 84.88) (width 1) (layer "B.Cu") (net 14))
 (segment (start 131.39 122.31) (end 131.36 122.34) (width 1) (layer "B.Cu") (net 7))
 (segment (start 138.16 122.31) (end 131.39 122.31) (width 1) (layer "B.Cu") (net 7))
 (segment (start 145.09 82.34) (end 145.09 84.88) (width 1) (layer "B.Cu") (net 15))
 (segment (start 144.39 122.01) (end 139.01 127.39) (width 1) (layer "B.Cu") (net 15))
 (segment (start 145.09 84.88) (end 144.39 85.58) (width 1) (layer "B.Cu") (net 15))
 (segment (start 144.39 85.58) (end 144.39 122.01) (width 1) (layer "B.Cu") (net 15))
 (segment (start 139.01 127.39) (end 138.16 127.39) (width 1) (layer "B.Cu") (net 15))
 (segment (start 170.23 94.9) (end 170.23 87.94) (width 1) (layer "B.Cu") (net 22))
 (segment (start 170.23 87.94) (end 174.55 83.62) (width 1) (layer "B.Cu") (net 22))
 (segment (start 162.885 102.555) (end 165.015 104.685) (width 1) (layer "B.Cu") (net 6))
 (segment (start 177.345 104.685) (end 179.39 106.73) (width 1) (layer "B.Cu") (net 6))
 (segment (start 179.39 110.22) (end 177.96 111.65) (width 1) (layer "B.Cu") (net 6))
 (segment (start 172.62 111.65) (end 168.14 116.13) (width 1) (layer "B.Cu") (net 6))
 (segment (start 168.14 116.13) (end 168.14 125.905) (width 1) (layer "B.Cu") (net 6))
 (segment (start 165.015 104.685) (end 173.145 104.685) (width 1) (layer "B.Cu") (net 6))
 (segment (start 177.96 111.65) (end 172.62 111.65) (width 1) (layer "B.Cu") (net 6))
 (segment (start 173.145 104.685) (end 177.345 104.685) (width 1) (layer "B.Cu") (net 6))
 (segment (start 179.39 106.73) (end 179.39 110.22) (width 1) (layer "B.Cu") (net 6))
 (segment (start 138.16 109.61) (end 137.31 109.61) (width 1) (layer "B.Cu") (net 19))
 (segment (start 132.42 104.72) (end 132.42 87.39) (width 1) (layer "B.Cu") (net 19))
 (segment (start 137.31 109.61) (end 132.42 104.72) (width 1) (layer "B.Cu") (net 19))
 (segment (start 134.93 82.34) (end 134.93 84.88) (width 1) (layer "B.Cu") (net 19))
 (segment (start 132.42 87.39) (end 134.93 84.88) (width 1) (layer "B.Cu") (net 19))
 (segment (start 130.98 117.9) (end 128.44 117.9) (width 1) (layer "B.Cu") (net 1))
 (segment (start 130.98 117.9) (end 133.97 117.9) (width 1) (layer "B.Cu") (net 1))
 (segment (start 133.97 117.9) (end 137.18 114.69) (width 1) (layer "B.Cu") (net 1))
 (segment (start 137.18 114.69) (end 138.16 114.69) (width 1) (layer "B.Cu") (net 1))
 (segment (start 167.34 111.145) (end 167.34 114.36) (width 1) (layer "B.Cu") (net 5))
 (segment (start 168.965 108.185) (end 166.675 110.475) (width 1) (layer "B.Cu") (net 5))
 (segment (start 166.675 110.48) (end 162.885 114.27) (width 1) (layer "B.Cu") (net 5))
 (segment (start 166.675 110.48) (end 167.34 111.145) (width 1) (layer "B.Cu") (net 5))
 (segment (start 173.145 108.185) (end 168.965 108.185) (width 1) (layer "B.Cu") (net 5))
 (segment (start 162.885 114.27) (end 162.885 115.255) (width 1) (layer "B.Cu") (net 5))
 (segment (start 166.675 110.475) (end 166.675 110.48) (width 1) (layer "B.Cu") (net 5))
 (segment (start 177.72 128.2) (end 177.72 125.37) (width 1) (layer "B.Cu") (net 8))
 (segment (start 173.98 132.24) (end 173.98 131.97) (width 1) (layer "B.Cu") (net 8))
 (segment (start 131.36 129.96) (end 137.28 135.88) (width 1) (layer "B.Cu") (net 8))
 (segment (start 170.34 135.88) (end 173.98 132.24) (width 1) (layer "B.Cu") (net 8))
 (segment (start 137.28 135.88) (end 170.34 135.88) (width 1) (layer "B.Cu") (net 8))
 (segment (start 173.98 131.94) (end 177.72 128.2) (width 1) (layer "B.Cu") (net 8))
 (segment (start 173.98 131.97) (end 173.98 131.94) (width 1) (layer "B.Cu") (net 8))
 (segment (start 178.99 121.76) (end 178.99 120.18) (width 1) (layer "B.Cu") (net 9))
 (segment (start 174.96 116.15) (end 176.68 117.87) (width 1) (layer "B.Cu") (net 9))
 (segment (start 178.99 125.37) (end 178.99 122.32) (width 1) (layer "B.Cu") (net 9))
 (segment (start 174.96 114.36) (end 174.96 116.15) (width 1) (layer "B.Cu") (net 9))
 (segment (start 178.99 120.18) (end 178.3 119.49) (width 1) (layer "B.Cu") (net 9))
 (segment (start 178.99 122.32) (end 178.99 121.76) (width 1) (layer "B.Cu") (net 9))
 (segment (start 176.68 117.87) (end 170.68 123.87) (width 1) (layer "B.Cu") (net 9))
 (segment (start 170.68 123.87) (end 170.68 125.905) (width 1) (layer "B.Cu") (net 9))
 (segment (start 176.68 117.87) (end 178.3 119.49) (width 1) (layer "B.Cu") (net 9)))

